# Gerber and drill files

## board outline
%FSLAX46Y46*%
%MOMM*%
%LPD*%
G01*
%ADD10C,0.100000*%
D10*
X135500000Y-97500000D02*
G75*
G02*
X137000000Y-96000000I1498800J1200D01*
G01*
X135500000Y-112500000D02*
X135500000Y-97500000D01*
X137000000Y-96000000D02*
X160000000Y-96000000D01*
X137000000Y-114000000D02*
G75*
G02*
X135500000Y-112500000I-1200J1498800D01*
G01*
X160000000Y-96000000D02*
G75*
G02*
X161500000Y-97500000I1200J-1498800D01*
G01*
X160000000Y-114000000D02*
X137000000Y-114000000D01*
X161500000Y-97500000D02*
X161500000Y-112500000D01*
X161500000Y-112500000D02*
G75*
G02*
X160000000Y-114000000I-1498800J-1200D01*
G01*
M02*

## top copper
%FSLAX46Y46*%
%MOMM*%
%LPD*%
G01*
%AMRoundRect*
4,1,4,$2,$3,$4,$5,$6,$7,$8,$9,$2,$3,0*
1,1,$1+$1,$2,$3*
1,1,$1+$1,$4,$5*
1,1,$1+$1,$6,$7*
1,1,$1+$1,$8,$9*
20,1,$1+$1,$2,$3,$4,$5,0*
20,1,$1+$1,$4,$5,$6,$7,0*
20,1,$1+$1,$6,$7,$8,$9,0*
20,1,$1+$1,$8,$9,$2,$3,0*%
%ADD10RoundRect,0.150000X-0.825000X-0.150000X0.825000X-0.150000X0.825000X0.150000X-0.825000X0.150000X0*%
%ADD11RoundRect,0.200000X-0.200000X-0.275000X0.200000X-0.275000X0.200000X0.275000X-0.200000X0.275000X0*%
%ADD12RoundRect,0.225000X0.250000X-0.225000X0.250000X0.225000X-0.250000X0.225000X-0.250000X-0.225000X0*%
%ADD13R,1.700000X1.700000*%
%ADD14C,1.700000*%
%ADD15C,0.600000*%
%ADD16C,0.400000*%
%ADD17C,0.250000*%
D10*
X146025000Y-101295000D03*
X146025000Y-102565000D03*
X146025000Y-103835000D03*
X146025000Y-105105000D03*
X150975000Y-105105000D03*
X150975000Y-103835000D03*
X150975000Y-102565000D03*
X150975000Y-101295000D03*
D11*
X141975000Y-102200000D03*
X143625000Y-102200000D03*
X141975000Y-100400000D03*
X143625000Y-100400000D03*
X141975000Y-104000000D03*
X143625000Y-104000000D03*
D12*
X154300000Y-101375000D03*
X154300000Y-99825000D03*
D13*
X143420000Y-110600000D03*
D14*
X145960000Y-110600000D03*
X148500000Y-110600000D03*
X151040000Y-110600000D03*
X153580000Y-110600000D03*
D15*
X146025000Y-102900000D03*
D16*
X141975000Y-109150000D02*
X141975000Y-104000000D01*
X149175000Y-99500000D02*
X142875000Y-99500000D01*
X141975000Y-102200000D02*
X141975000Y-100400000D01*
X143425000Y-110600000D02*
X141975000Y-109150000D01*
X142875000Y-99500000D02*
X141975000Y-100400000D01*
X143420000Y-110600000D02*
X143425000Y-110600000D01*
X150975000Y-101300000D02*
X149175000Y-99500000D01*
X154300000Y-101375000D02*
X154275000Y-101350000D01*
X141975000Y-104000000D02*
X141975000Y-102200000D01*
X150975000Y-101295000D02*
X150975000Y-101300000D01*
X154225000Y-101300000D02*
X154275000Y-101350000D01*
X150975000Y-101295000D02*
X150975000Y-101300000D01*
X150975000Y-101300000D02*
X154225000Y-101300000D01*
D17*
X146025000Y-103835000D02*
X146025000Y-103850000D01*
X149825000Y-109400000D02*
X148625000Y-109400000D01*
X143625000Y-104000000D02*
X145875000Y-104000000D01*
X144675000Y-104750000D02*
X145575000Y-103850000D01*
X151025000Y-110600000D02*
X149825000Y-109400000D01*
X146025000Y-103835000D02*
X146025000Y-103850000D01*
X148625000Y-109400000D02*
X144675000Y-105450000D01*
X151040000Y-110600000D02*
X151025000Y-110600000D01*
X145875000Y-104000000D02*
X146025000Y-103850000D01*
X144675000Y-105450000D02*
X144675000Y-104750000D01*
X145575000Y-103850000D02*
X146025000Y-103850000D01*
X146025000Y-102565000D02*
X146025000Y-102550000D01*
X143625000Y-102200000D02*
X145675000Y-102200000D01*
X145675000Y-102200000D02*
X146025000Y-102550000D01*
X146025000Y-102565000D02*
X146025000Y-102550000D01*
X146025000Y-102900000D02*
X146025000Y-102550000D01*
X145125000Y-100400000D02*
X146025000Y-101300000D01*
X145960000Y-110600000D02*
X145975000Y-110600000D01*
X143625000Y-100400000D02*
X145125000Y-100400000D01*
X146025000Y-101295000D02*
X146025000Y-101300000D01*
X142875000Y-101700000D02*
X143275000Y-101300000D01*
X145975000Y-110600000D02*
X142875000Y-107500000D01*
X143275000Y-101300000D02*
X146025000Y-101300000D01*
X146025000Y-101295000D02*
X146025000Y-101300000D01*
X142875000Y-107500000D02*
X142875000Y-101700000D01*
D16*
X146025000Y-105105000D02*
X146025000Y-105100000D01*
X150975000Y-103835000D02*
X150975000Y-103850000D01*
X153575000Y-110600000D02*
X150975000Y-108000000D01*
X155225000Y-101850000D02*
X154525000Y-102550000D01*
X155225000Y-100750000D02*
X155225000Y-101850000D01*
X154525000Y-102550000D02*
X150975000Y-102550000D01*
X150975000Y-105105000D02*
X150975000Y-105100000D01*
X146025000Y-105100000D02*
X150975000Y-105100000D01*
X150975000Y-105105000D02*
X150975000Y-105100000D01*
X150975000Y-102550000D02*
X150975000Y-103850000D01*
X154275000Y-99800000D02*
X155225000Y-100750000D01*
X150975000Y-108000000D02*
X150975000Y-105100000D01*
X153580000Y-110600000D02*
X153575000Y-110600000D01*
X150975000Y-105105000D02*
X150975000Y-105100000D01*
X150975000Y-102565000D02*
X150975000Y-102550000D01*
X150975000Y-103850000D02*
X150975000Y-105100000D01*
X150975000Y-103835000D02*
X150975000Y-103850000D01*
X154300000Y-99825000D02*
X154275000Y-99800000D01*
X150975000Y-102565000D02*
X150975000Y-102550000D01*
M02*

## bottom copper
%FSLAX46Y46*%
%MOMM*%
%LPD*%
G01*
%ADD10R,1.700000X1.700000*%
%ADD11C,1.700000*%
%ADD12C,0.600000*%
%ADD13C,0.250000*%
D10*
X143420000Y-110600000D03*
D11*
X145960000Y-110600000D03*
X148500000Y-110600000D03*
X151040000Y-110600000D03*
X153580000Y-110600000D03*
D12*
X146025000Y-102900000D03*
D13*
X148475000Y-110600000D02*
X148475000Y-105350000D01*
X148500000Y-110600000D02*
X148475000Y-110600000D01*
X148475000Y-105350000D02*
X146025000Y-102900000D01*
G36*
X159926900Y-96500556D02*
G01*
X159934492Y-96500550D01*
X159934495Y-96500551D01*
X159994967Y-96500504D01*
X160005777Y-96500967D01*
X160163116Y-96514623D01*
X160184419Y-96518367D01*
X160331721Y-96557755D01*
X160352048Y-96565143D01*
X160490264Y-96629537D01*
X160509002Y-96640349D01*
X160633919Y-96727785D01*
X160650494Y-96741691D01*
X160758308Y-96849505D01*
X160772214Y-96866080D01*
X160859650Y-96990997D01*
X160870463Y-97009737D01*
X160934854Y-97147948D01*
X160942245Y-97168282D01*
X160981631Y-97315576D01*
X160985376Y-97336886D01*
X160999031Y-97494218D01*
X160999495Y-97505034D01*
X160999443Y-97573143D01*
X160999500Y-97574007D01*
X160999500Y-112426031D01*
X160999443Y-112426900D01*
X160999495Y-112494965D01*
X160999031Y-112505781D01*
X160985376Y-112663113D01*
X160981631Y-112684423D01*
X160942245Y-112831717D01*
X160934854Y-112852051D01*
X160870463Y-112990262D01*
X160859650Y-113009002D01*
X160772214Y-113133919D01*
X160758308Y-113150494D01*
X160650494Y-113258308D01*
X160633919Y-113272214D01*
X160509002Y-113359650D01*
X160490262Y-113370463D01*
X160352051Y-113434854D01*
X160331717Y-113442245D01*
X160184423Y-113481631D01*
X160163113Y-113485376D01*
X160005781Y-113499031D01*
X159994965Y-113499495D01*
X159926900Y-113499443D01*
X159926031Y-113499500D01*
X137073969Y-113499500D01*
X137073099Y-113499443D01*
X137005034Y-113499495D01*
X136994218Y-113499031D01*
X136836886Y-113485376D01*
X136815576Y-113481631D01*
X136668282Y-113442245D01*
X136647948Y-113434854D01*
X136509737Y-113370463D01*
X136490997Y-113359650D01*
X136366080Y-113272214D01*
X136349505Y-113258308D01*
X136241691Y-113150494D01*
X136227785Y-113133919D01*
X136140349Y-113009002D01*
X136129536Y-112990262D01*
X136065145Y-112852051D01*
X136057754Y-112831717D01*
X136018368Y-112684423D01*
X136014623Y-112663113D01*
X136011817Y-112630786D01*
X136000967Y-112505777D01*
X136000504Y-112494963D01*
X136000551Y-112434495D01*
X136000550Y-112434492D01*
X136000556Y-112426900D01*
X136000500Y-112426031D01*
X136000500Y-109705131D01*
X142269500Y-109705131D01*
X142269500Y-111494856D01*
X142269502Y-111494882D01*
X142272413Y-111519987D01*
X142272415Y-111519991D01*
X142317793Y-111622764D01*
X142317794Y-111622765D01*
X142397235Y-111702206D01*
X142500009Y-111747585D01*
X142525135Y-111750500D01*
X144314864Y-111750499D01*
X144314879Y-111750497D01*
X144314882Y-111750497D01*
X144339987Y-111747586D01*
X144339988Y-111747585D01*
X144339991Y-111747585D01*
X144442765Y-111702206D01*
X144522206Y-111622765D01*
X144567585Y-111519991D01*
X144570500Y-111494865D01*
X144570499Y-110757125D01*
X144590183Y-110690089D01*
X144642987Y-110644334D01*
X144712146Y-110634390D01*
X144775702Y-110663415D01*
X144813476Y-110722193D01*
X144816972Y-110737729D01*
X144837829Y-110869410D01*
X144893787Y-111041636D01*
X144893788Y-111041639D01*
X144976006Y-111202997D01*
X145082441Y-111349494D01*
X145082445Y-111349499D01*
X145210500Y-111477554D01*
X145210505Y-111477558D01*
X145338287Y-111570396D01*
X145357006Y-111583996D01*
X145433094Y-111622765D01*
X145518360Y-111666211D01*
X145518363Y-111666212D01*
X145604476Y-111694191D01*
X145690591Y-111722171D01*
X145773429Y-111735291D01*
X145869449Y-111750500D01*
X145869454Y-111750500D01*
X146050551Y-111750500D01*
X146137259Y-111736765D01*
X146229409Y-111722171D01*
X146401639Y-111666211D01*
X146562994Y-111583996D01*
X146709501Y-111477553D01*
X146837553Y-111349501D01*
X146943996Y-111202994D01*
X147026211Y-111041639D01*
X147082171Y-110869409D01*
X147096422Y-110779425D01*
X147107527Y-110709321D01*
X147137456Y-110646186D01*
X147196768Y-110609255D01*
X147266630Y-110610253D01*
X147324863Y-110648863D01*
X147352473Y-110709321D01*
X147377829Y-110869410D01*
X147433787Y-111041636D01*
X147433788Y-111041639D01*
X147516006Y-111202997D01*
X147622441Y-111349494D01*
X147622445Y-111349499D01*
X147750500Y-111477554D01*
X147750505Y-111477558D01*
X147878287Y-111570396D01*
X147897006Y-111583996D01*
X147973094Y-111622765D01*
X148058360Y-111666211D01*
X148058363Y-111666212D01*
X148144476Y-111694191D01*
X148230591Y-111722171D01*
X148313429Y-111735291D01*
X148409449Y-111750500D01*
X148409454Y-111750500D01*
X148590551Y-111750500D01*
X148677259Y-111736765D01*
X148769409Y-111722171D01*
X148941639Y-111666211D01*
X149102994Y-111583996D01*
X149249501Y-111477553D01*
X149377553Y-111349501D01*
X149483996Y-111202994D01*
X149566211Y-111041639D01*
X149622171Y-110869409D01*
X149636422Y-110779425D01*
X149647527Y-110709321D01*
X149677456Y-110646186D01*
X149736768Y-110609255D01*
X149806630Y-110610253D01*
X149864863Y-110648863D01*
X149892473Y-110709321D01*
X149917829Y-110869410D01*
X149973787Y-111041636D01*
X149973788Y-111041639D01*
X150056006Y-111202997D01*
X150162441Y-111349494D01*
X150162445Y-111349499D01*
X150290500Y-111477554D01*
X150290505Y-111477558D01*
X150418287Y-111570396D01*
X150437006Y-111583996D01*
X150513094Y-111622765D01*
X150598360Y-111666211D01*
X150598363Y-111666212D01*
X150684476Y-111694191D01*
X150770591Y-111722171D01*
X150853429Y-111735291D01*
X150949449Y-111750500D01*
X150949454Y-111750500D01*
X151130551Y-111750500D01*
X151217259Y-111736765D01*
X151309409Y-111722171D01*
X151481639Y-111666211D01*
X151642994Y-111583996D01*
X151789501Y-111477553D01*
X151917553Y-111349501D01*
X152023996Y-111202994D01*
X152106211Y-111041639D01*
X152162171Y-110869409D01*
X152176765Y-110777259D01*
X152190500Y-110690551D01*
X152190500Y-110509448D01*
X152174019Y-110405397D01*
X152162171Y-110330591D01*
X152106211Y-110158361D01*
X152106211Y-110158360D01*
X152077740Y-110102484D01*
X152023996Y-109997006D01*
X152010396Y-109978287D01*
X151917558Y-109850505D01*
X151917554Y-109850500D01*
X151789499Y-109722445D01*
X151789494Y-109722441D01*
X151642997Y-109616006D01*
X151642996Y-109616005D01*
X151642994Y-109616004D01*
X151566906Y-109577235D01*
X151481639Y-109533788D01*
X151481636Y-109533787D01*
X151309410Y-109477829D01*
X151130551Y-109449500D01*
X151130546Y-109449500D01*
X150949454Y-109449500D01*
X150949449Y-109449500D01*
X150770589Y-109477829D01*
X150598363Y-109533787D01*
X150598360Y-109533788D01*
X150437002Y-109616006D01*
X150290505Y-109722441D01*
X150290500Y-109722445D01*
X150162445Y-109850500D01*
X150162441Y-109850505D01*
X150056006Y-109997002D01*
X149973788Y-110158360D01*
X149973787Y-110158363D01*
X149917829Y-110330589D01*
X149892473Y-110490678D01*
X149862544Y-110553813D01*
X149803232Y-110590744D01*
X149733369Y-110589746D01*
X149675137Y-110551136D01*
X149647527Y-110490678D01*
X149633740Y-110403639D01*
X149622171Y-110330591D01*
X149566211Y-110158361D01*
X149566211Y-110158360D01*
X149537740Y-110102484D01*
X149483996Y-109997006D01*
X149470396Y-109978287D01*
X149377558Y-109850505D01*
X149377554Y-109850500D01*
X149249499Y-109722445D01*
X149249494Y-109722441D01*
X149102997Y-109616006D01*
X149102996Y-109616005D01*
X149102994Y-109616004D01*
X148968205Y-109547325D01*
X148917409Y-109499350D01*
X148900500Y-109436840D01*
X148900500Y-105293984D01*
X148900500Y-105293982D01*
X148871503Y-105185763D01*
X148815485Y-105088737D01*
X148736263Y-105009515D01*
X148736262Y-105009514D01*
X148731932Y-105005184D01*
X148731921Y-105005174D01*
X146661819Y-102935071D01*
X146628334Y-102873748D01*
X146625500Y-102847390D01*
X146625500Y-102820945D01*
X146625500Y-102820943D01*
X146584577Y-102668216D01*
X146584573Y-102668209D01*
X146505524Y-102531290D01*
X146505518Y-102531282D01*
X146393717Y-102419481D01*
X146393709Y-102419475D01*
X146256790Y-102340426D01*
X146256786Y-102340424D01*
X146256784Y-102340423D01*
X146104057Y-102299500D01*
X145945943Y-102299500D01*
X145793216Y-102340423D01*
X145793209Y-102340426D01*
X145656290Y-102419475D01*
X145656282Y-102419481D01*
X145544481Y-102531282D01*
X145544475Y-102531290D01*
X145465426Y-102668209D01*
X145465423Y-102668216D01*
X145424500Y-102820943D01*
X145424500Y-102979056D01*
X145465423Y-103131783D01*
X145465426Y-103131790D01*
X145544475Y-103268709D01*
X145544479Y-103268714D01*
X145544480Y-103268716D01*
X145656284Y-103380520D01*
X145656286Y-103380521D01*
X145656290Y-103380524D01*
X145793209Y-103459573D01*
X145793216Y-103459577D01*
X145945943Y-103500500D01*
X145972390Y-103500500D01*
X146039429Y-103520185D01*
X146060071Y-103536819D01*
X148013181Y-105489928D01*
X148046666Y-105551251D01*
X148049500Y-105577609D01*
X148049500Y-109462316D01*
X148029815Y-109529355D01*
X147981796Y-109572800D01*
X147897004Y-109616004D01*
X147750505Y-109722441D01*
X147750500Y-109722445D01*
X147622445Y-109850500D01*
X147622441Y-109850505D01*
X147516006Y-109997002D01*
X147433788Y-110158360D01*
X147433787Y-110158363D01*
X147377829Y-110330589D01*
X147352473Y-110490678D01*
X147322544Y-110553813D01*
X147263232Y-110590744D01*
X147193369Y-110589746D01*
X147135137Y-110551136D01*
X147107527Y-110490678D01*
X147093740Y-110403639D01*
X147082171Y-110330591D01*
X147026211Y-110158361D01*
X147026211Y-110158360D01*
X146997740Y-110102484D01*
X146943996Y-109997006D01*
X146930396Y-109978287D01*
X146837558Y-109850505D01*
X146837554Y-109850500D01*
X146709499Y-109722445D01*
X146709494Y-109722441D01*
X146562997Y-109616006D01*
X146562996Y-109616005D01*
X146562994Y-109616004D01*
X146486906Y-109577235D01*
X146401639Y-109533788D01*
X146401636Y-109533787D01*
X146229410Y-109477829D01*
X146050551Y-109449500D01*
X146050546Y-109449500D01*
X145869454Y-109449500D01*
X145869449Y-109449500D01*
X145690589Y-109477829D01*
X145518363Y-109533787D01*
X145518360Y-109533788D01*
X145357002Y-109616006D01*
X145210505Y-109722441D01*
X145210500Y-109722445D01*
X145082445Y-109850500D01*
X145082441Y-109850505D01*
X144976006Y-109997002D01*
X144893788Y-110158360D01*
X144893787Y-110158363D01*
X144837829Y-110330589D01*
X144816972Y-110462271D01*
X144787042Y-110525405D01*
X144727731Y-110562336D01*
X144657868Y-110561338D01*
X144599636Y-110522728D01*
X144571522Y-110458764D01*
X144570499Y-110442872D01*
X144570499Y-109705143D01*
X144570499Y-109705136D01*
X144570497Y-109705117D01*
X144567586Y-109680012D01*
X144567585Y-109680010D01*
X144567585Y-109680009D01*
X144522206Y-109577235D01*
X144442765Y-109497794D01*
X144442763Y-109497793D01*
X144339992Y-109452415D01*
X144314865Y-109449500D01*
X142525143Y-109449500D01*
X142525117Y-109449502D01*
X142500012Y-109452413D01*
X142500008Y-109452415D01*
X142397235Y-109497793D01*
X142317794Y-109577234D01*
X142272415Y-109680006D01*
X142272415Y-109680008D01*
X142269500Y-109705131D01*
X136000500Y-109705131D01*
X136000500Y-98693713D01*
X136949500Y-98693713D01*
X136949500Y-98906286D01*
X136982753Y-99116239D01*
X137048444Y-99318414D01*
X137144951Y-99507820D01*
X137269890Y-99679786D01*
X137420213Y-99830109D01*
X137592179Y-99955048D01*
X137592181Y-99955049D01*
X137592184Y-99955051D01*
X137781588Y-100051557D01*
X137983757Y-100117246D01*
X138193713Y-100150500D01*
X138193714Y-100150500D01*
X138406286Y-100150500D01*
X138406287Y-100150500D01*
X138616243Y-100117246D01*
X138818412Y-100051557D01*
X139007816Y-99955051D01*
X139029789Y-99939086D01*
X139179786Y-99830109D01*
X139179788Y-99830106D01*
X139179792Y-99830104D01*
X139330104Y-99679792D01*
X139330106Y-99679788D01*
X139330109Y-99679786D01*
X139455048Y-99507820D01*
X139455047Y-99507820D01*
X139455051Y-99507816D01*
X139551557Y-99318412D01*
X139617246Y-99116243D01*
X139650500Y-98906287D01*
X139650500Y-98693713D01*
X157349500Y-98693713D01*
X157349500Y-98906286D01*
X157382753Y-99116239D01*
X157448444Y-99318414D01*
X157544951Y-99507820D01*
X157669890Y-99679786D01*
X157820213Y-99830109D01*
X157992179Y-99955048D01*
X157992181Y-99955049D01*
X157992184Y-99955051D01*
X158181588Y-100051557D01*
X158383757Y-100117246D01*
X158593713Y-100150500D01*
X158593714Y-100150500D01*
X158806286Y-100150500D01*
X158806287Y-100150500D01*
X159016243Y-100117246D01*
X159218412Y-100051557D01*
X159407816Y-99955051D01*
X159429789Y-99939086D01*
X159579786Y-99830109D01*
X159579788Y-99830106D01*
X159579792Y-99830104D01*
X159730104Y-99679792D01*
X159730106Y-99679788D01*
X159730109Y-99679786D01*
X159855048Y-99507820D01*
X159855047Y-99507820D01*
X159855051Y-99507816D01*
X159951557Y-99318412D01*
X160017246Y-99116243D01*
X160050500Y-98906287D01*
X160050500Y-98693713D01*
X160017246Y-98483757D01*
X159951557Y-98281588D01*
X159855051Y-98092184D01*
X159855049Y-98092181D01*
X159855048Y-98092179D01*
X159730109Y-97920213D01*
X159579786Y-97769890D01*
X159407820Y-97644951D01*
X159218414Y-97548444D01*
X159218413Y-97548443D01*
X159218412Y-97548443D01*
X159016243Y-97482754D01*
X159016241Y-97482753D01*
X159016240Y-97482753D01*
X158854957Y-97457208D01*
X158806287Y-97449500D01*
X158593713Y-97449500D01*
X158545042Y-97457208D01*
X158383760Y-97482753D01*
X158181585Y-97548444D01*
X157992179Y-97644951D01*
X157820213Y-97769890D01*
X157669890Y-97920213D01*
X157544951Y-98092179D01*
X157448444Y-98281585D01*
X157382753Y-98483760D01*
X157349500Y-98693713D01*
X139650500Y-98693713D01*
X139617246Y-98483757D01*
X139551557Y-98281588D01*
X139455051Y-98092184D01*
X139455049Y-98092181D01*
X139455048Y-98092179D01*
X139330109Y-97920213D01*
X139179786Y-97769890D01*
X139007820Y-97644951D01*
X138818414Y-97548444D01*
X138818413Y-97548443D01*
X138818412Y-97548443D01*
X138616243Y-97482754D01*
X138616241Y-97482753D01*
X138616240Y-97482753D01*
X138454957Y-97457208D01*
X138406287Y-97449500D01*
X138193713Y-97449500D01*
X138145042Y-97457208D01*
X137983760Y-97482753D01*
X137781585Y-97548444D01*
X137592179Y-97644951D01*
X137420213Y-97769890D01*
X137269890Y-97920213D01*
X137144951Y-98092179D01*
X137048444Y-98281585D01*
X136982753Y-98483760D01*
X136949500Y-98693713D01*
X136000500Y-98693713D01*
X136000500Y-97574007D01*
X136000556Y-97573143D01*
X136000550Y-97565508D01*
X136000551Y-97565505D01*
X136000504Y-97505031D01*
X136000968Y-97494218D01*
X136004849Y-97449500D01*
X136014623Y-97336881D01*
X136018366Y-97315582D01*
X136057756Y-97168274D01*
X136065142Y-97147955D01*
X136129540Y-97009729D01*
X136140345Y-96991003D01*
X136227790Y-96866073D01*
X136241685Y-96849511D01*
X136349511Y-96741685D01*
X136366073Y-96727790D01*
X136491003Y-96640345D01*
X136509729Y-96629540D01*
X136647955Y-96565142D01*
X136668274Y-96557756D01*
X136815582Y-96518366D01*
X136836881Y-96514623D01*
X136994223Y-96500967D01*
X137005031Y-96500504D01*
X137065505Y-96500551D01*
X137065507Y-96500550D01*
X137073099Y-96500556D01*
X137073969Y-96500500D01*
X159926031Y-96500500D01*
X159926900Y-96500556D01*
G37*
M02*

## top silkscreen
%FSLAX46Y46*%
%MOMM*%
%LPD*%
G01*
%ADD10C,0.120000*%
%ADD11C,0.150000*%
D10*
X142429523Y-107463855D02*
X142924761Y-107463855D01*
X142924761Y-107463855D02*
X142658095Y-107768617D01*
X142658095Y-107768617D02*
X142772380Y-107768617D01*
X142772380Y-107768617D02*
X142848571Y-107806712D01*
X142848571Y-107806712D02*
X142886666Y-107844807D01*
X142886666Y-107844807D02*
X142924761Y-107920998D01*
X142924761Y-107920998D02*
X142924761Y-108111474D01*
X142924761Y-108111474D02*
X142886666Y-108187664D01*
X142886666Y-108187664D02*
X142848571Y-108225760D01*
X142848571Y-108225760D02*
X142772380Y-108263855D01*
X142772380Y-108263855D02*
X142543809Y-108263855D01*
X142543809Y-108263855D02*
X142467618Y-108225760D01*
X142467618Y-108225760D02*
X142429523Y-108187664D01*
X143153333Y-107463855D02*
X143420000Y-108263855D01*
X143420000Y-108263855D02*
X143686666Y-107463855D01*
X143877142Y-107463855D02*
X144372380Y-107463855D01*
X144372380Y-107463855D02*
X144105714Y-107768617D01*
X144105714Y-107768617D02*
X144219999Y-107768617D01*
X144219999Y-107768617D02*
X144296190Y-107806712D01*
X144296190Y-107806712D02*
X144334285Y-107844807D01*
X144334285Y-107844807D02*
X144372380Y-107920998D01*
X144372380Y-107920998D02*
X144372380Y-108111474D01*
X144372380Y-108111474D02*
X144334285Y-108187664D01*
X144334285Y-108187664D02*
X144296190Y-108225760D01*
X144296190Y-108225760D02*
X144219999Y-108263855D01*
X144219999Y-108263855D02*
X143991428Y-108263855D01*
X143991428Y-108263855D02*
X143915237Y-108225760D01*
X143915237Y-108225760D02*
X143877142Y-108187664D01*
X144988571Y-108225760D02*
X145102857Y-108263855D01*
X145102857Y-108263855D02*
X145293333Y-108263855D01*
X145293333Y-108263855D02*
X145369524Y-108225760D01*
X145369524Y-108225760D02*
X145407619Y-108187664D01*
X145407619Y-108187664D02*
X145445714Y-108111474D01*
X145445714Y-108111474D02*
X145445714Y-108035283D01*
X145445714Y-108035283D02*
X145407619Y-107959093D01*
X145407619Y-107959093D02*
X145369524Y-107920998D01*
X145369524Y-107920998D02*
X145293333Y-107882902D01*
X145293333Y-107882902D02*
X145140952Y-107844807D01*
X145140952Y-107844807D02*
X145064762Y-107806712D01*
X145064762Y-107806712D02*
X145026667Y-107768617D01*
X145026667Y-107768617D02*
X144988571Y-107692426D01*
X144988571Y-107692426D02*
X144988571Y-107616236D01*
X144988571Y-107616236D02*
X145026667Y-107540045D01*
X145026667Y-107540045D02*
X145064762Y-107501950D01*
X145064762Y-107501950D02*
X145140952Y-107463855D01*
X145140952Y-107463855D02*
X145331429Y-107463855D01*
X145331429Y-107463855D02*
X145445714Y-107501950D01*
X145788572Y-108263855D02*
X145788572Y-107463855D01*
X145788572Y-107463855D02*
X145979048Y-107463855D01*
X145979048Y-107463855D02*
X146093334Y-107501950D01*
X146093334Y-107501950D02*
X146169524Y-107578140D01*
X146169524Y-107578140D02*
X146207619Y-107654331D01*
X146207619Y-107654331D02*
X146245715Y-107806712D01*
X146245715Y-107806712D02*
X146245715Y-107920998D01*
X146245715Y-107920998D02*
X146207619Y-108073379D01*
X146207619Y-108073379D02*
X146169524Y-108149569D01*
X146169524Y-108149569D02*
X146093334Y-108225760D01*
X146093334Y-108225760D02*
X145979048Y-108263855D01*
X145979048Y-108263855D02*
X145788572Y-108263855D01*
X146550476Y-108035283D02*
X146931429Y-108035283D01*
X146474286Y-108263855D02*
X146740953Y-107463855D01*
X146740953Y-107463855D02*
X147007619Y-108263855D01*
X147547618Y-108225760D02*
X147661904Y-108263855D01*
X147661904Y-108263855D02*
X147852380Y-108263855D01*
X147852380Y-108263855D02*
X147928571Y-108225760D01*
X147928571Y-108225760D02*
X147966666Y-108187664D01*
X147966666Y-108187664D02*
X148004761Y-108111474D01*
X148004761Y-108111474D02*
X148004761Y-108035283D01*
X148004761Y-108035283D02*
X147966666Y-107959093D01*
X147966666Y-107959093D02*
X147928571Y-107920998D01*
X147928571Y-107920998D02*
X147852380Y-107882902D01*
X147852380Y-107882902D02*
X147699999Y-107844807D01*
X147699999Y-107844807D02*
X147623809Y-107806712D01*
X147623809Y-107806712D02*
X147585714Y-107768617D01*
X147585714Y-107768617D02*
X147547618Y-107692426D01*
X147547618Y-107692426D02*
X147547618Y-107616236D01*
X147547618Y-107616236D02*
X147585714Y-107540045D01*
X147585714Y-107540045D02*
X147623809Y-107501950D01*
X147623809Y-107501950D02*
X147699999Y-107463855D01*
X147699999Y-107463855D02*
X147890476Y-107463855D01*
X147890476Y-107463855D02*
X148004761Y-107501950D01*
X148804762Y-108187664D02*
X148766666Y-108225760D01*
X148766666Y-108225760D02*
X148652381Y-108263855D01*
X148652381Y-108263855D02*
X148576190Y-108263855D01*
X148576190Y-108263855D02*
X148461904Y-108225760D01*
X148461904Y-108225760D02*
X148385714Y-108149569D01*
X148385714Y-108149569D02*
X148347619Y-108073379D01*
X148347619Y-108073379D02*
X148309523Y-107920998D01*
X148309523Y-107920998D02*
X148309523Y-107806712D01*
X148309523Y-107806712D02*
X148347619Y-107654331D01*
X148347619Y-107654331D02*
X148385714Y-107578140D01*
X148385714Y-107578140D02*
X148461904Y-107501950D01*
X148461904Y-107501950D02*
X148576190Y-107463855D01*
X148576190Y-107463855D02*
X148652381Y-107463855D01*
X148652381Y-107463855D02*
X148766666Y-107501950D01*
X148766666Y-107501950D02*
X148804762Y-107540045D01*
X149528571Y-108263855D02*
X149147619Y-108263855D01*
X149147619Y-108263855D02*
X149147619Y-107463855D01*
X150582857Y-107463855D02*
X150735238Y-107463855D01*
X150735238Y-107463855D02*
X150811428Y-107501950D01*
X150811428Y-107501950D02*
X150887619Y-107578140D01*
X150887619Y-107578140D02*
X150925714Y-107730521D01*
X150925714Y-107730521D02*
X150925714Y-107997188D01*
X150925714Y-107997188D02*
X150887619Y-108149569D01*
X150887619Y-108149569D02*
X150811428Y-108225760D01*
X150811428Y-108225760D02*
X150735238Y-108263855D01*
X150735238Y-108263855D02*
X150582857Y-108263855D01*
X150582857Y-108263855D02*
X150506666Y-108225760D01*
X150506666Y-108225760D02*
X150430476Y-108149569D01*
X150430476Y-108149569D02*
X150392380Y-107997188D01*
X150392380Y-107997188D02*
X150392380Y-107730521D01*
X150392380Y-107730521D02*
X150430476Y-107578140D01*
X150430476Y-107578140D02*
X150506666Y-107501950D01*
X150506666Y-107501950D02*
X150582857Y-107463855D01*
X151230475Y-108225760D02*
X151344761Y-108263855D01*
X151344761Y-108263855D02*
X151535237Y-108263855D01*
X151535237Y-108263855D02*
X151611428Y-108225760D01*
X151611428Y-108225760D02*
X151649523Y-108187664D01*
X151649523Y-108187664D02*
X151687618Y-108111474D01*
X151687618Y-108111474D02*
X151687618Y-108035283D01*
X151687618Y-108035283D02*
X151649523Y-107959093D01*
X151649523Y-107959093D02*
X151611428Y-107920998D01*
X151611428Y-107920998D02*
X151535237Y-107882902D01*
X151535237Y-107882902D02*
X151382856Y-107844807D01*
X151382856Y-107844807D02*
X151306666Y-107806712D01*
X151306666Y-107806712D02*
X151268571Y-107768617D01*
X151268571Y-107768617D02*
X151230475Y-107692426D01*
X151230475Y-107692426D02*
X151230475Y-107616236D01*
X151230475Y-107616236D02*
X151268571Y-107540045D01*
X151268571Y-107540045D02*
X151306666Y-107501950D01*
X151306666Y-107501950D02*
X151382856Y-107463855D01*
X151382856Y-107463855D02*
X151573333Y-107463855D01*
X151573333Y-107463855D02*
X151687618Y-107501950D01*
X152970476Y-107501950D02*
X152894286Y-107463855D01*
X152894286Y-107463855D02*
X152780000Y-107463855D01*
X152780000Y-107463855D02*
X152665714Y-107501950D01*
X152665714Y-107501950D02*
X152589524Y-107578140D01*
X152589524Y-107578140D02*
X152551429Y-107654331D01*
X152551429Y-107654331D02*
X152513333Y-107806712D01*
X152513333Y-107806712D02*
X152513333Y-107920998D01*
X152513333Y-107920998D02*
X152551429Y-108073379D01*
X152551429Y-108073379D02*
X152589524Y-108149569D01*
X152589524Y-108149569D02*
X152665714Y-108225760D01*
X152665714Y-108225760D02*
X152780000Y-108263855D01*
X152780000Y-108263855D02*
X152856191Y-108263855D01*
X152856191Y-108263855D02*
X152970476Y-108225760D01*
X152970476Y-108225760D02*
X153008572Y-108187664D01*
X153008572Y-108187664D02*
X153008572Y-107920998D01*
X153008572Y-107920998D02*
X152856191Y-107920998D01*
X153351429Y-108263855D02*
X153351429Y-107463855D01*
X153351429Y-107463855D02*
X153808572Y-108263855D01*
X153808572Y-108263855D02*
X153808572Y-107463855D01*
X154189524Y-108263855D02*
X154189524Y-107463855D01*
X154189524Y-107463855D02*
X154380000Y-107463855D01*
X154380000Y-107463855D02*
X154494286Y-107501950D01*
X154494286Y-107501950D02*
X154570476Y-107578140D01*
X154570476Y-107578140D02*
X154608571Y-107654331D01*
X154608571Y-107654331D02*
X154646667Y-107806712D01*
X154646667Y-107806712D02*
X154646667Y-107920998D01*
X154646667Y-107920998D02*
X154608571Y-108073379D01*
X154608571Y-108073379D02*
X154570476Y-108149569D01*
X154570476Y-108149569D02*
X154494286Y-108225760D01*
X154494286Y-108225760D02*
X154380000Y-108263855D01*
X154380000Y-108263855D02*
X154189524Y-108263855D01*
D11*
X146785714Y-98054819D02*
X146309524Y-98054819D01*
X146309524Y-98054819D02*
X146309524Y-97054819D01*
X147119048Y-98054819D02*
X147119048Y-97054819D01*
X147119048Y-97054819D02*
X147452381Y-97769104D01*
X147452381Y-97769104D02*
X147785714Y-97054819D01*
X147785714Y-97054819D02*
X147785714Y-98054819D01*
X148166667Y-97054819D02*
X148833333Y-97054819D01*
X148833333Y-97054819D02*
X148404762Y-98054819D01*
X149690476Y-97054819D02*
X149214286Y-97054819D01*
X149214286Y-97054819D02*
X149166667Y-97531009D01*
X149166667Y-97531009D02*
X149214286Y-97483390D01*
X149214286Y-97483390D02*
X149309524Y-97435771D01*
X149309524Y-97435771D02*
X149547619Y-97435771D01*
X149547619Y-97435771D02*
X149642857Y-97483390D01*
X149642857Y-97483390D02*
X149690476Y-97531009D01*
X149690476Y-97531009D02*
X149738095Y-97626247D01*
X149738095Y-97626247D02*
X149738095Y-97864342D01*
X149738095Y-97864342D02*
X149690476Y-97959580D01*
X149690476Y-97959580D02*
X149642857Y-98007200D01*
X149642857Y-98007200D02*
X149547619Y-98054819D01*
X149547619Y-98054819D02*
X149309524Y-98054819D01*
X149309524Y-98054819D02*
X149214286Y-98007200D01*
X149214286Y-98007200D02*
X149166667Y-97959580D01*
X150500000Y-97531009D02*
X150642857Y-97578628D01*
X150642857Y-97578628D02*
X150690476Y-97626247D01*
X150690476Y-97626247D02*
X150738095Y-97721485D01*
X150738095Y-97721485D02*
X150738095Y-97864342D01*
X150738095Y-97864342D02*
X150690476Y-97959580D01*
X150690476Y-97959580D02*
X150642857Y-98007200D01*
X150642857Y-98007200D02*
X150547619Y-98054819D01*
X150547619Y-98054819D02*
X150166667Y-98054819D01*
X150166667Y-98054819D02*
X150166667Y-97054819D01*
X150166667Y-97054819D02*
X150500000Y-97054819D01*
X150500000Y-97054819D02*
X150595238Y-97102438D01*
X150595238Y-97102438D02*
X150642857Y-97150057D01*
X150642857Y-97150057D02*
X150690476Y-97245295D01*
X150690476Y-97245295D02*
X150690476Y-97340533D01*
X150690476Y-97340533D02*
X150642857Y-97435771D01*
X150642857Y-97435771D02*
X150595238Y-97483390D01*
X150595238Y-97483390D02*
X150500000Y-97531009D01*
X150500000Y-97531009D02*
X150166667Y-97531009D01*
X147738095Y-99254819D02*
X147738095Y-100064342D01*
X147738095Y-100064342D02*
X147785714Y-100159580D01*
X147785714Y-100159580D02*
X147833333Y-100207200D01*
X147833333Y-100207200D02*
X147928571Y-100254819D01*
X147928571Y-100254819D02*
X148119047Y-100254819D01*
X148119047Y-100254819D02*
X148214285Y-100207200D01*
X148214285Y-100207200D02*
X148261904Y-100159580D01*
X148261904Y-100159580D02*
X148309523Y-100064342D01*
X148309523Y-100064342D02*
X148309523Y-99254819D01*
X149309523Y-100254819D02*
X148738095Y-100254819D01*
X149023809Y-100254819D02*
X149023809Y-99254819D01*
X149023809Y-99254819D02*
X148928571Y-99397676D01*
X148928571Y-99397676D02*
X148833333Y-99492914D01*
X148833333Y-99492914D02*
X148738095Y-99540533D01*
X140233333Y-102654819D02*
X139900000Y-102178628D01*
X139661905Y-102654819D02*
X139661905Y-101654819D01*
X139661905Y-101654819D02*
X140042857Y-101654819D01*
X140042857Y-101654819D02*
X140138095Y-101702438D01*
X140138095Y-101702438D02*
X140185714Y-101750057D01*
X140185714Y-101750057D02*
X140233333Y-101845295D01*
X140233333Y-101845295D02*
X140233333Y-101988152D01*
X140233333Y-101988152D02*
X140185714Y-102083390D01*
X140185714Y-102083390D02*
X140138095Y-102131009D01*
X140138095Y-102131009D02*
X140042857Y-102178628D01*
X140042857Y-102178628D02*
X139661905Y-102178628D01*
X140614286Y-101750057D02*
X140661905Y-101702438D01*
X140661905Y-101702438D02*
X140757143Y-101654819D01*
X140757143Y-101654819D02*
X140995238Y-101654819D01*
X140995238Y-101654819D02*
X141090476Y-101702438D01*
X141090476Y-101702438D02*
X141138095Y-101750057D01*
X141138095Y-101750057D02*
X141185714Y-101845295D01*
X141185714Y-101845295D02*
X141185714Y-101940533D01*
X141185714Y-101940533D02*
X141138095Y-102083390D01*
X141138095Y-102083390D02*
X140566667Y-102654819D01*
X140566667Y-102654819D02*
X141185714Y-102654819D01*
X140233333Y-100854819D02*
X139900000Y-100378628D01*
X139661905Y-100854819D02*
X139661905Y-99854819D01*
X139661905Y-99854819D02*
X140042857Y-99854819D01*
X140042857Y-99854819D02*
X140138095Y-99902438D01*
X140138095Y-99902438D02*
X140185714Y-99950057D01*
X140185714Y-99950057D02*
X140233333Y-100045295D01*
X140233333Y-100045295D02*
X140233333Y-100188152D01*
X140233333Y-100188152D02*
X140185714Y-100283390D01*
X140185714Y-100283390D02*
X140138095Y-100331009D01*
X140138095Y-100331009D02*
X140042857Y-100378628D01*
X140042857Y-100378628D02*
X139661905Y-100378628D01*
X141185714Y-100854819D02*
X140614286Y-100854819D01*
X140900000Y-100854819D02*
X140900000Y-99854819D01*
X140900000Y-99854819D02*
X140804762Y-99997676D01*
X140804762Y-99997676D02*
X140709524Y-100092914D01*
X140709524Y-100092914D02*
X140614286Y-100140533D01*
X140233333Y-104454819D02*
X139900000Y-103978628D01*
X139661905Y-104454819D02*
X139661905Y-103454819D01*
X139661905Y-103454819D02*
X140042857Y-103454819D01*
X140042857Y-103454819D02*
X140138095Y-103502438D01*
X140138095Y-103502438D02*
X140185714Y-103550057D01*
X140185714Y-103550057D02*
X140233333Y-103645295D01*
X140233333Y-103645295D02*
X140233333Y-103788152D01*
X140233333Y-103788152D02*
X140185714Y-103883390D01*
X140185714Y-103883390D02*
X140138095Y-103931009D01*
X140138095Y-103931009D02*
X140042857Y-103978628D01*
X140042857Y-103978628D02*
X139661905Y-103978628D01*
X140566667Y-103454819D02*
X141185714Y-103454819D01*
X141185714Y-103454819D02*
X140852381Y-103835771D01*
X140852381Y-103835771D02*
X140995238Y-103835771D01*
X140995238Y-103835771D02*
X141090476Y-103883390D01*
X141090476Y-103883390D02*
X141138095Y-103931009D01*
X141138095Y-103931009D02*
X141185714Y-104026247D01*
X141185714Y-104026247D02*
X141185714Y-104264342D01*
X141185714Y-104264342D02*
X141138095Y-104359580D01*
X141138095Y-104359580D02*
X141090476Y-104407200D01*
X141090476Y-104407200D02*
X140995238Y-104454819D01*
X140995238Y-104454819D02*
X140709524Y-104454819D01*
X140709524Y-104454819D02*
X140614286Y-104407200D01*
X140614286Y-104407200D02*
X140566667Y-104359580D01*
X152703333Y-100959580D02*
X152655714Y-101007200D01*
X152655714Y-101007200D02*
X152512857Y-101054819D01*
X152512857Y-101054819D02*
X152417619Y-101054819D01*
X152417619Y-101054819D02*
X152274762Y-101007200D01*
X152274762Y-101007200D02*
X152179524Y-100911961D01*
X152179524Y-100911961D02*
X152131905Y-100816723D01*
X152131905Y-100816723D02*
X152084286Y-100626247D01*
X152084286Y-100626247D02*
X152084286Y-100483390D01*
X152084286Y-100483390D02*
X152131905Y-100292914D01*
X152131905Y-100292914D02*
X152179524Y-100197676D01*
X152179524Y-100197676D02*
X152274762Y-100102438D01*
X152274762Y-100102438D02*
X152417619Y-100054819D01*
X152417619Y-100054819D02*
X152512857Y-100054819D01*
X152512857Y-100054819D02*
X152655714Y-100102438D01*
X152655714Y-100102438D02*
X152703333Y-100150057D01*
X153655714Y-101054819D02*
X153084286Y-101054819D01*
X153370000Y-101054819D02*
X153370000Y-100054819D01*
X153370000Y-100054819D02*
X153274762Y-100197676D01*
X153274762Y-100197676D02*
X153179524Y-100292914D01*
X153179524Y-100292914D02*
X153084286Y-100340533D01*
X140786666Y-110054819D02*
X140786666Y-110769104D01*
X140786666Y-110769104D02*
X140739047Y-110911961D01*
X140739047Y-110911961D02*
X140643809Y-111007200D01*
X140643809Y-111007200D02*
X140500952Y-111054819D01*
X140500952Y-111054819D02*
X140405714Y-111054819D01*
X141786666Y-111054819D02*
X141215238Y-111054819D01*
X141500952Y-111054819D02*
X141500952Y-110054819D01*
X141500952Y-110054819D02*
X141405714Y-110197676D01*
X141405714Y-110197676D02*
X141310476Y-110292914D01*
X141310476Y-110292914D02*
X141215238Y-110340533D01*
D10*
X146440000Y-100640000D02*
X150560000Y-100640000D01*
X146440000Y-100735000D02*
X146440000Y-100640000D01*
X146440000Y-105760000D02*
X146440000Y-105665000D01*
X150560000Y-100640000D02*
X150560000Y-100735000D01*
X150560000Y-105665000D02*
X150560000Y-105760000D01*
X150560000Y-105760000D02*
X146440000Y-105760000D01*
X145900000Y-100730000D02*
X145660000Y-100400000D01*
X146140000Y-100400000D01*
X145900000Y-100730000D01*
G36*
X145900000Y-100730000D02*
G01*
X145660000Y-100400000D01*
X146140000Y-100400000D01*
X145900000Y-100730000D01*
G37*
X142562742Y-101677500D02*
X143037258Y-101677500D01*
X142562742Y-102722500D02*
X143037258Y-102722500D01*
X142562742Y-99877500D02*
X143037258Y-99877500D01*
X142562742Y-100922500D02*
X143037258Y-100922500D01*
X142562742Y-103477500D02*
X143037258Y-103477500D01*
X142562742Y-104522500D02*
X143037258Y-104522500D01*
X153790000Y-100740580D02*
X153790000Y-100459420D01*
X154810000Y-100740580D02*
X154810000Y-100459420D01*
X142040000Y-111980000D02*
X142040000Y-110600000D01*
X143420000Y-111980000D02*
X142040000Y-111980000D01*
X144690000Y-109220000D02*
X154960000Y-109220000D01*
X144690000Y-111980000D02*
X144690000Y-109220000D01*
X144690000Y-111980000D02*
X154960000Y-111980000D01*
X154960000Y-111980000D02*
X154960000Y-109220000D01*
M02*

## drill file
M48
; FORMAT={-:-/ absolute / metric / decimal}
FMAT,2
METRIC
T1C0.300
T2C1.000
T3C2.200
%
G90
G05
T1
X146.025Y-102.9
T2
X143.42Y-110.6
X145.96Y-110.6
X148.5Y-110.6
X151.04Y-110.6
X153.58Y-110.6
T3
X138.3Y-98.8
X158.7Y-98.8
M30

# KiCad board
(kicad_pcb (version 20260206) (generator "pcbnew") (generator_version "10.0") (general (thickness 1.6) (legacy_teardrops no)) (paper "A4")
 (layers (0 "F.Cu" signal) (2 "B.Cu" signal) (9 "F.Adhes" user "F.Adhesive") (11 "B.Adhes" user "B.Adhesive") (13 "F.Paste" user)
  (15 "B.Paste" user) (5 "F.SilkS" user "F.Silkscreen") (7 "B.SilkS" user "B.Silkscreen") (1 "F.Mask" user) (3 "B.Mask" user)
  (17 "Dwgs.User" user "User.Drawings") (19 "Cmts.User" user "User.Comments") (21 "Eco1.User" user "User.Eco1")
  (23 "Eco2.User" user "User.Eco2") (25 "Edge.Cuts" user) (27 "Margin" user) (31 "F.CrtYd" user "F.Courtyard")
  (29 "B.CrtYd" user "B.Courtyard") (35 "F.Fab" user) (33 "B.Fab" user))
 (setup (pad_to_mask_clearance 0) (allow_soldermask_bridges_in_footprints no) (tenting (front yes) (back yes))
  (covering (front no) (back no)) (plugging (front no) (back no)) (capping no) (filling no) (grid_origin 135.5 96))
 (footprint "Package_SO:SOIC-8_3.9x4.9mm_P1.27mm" (layer "F.Cu") (at 148.5 103.2)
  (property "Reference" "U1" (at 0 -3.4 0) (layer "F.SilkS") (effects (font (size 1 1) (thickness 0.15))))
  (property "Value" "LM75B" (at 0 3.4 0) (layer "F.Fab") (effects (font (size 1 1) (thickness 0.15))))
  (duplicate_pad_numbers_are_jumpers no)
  (fp_line (start -2.06 -2.56) (end 2.06 -2.56) (stroke (width 0.12) (type solid)) (layer "F.SilkS"))
  (fp_line (start -2.06 -2.465) (end -2.06 -2.56) (stroke (width 0.12) (type solid)) (layer "F.SilkS"))
  (fp_line (start -2.06 2.56) (end -2.06 2.465) (stroke (width 0.12) (type solid)) (layer "F.SilkS"))
  (fp_line (start 2.06 -2.56) (end 2.06 -2.465) (stroke (width 0.12) (type solid)) (layer "F.SilkS"))
  (fp_line (start 2.06 2.465) (end 2.06 2.56) (stroke (width 0.12) (type solid)) (layer "F.SilkS"))
  (fp_line (start 2.06 2.56) (end -2.06 2.56) (stroke (width 0.12) (type solid)) (layer "F.SilkS"))
  (fp_poly (pts (xy -2.6 -2.47) (xy -2.84 -2.8) (xy -2.36 -2.8)) (stroke (width 0.12) (type solid)) (fill yes) (layer "F.SilkS"))
  (pad "1" smd roundrect (at -2.475 -1.905) (size 1.95 0.6) (layers "F.Cu" "F.Mask" "F.Paste") (roundrect_rratio 0.25) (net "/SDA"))
  (pad "2" smd roundrect (at -2.475 -0.635) (size 1.95 0.6) (layers "F.Cu" "F.Mask" "F.Paste") (roundrect_rratio 0.25) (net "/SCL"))
  (pad "3" smd roundrect (at -2.475 0.635) (size 1.95 0.6) (layers "F.Cu" "F.Mask" "F.Paste") (roundrect_rratio 0.25) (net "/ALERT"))
  (pad "4" smd roundrect (at -2.475 1.905) (size 1.95 0.6) (layers "F.Cu" "F.Mask" "F.Paste") (roundrect_rratio 0.25) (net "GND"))
  (pad "5" smd roundrect (at 2.475 1.905) (size 1.95 0.6) (layers "F.Cu" "F.Mask" "F.Paste") (roundrect_rratio 0.25) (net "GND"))
  (pad "6" smd roundrect (at 2.475 0.635) (size 1.95 0.6) (layers "F.Cu" "F.Mask" "F.Paste") (roundrect_rratio 0.25) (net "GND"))
  (pad "7" smd roundrect (at 2.475 -0.635) (size 1.95 0.6) (layers "F.Cu" "F.Mask" "F.Paste") (roundrect_rratio 0.25) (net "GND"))
  (pad "8" smd roundrect (at 2.475 -1.905) (size 1.95 0.6) (layers "F.Cu" "F.Mask" "F.Paste") (roundrect_rratio 0.25) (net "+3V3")))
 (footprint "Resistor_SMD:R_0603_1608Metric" (layer "F.Cu") (at 142.8 102.2)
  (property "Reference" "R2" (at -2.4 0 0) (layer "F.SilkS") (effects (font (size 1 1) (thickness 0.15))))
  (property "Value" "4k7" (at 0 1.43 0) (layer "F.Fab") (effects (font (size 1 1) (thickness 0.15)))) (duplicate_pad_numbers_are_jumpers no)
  (fp_line (start -0.237258 -0.5225) (end 0.237258 -0.5225) (stroke (width 0.12) (type solid)) (layer "F.SilkS"))
  (fp_line (start -0.237258 0.5225) (end 0.237258 0.5225) (stroke (width 0.12) (type solid)) (layer "F.SilkS"))
  (pad "1" smd roundrect (at -0.825 0) (size 0.8 0.95) (layers "F.Cu" "F.Mask" "F.Paste") (roundrect_rratio 0.25) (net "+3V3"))
  (pad "2" smd roundrect (at 0.825 0) (size 0.8 0.95) (layers "F.Cu" "F.Mask" "F.Paste") (roundrect_rratio 0.25) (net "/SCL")))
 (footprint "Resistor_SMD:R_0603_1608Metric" (layer "F.Cu") (at 142.8 100.4)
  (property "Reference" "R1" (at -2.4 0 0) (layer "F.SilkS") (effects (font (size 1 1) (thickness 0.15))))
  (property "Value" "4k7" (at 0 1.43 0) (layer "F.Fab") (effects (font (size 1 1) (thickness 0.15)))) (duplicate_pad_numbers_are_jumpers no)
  (fp_line (start -0.237258 -0.5225) (end 0.237258 -0.5225) (stroke (width 0.12) (type solid)) (layer "F.SilkS"))
  (fp_line (start -0.237258 0.5225) (end 0.237258 0.5225) (stroke (width 0.12) (type solid)) (layer "F.SilkS"))
  (pad "1" smd roundrect (at -0.825 0) (size 0.8 0.95) (layers "F.Cu" "F.Mask" "F.Paste") (roundrect_rratio 0.25) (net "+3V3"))
  (pad "2" smd roundrect (at 0.825 0) (size 0.8 0.95) (layers "F.Cu" "F.Mask" "F.Paste") (roundrect_rratio 0.25) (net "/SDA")))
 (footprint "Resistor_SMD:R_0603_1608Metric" (layer "F.Cu") (at 142.8 104)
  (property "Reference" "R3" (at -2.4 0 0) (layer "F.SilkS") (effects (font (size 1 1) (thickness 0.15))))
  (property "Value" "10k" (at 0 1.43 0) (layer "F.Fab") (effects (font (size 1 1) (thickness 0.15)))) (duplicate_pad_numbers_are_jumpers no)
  (fp_line (start -0.237258 -0.5225) (end 0.237258 -0.5225) (stroke (width 0.12) (type solid)) (layer "F.SilkS"))
  (fp_line (start -0.237258 0.5225) (end 0.237258 0.5225) (stroke (width 0.12) (type solid)) (layer "F.SilkS"))
  (pad "1" smd roundrect (at -0.825 0) (size 0.8 0.95) (layers "F.Cu" "F.Mask" "F.Paste") (roundrect_rratio 0.25) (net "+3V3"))
  (pad "2" smd roundrect (at 0.825 0) (size 0.8 0.95) (layers "F.Cu" "F.Mask" "F.Paste") (roundrect_rratio 0.25) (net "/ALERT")))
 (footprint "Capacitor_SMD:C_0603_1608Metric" (layer "F.Cu") (at 154.3 100.6 90)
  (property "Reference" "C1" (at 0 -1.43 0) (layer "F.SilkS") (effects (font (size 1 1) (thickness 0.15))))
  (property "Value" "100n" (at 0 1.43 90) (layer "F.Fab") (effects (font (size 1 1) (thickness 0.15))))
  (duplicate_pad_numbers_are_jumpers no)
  (fp_line (start -0.14058 -0.51) (end 0.14058 -0.51) (stroke (width 0.12) (type solid)) (layer "F.SilkS"))
  (fp_line (start -0.14058 0.51) (end 0.14058 0.51) (stroke (width 0.12) (type solid)) (layer "F.SilkS"))
  (pad "1" smd roundrect (at -0.775 0 90) (size 0.9 0.95) (layers "F.Cu" "F.Mask" "F.Paste") (roundrect_rratio 0.25) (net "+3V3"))
  (pad "2" smd roundrect (at 0.775 0 90) (size 0.9 0.95) (layers "F.Cu" "F.Mask" "F.Paste") (roundrect_rratio 0.25) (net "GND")))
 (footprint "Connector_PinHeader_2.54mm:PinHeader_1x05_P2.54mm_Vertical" (layer "F.Cu") (at 143.42 110.6 90)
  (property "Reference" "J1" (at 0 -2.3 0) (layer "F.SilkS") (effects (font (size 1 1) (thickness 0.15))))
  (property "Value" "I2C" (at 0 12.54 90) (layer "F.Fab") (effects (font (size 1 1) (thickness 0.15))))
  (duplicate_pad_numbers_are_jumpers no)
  (fp_line (start -1.38 -1.38) (end 0 -1.38) (stroke (width 0.12) (type solid)) (layer "F.SilkS"))
  (fp_line (start -1.38 0) (end -1.38 -1.38) (stroke (width 0.12) (type solid)) (layer "F.SilkS"))
  (fp_line (start 1.38 1.27) (end 1.38 11.54) (stroke (width 0.12) (type solid)) (layer "F.SilkS"))
  (fp_line (start -1.38 1.27) (end 1.38 1.27) (stroke (width 0.12) (type solid)) (layer "F.SilkS"))
  (fp_line (start -1.38 1.27) (end -1.38 11.54) (stroke (width 0.12) (type solid)) (layer "F.SilkS"))
  (fp_line (start -1.38 11.54) (end 1.38 11.54) (stroke (width 0.12) (type solid)) (layer "F.SilkS"))
  (pad "1" thru_hole rect (at 0 0 90) (size 1.7 1.7) (drill 1) (layers "*.Cu" "*.Mask") (remove_unused_layers no) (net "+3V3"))
  (pad "2" thru_hole circle (at 0 2.54 90) (size 1.7 1.7) (drill 1) (layers "*.Cu" "*.Mask") (remove_unused_layers no) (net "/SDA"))
  (pad "3" thru_hole circle (at 0 5.08 90) (size 1.7 1.7) (drill 1) (layers "*.Cu" "*.Mask") (remove_unused_layers no) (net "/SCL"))
  (pad "4" thru_hole circle (at 0 7.62 90) (size 1.7 1.7) (drill 1) (layers "*.Cu" "*.Mask") (remove_unused_layers no) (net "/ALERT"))
  (pad "5" thru_hole circle (at 0 10.16 90) (size 1.7 1.7) (drill 1) (layers "*.Cu" "*.Mask") (remove_unused_layers no) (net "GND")))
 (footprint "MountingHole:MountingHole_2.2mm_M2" (layer "F.Cu") (at 138.3 98.8)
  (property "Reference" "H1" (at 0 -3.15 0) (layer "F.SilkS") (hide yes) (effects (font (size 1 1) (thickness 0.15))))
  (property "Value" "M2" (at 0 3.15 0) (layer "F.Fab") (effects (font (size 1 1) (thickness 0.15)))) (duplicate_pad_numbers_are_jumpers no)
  (pad "" np_thru_hole circle (at 0 0) (size 2.2 2.2) (drill 2.2) (layers "*.Cu" "*.Mask")))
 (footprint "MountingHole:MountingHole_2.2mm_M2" (layer "F.Cu") (at 158.7 98.8)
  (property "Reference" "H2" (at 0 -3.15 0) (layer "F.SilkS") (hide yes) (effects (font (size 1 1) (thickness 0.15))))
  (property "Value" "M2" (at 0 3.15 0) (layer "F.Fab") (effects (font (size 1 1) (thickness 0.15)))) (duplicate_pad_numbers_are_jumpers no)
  (pad "" np_thru_hole circle (at 0 0) (size 2.2 2.2) (drill 2.2) (layers "*.Cu" "*.Mask")))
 (gr_arc (start 135.5 97.5) (mid 135.939 96.439) (end 137 96) (stroke (width 0.1) (type default)) (layer "Edge.Cuts"))
 (gr_line (start 135.5 112.5) (end 135.5 97.5) (stroke (width 0.1) (type default)) (layer "Edge.Cuts"))
 (gr_line (start 137 96) (end 160 96) (stroke (width 0.1) (type default)) (layer "Edge.Cuts"))
 (gr_arc (start 137 114) (mid 135.939 113.561) (end 135.5 112.5) (stroke (width 0.1) (type default)) (layer "Edge.Cuts"))
 (gr_arc (start 160 96) (mid 161.061 96.439) (end 161.5 97.5) (stroke (width 0.1) (type default)) (layer "Edge.Cuts"))
 (gr_line (start 160 114) (end 137 114) (stroke (width 0.1) (type default)) (layer "Edge.Cuts"))
 (gr_line (start 161.5 97.5) (end 161.5 112.5) (stroke (width 0.1) (type default)) (layer "Edge.Cuts"))
 (gr_arc (start 161.5 112.5) (mid 161.061 113.561) (end 160 114) (stroke (width 0.1) (type default)) (layer "Edge.Cuts"))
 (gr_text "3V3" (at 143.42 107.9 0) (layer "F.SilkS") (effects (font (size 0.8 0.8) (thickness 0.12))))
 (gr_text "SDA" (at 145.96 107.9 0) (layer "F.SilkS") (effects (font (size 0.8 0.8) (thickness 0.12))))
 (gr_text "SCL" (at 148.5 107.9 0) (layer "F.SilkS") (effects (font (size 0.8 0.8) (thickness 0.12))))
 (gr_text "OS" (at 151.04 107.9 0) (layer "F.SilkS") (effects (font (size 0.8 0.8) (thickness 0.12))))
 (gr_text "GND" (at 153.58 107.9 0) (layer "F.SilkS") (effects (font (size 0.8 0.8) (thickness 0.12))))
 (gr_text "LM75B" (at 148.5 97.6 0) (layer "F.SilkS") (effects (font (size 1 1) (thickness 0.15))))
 (segment (start 141.975 109.15) (end 141.975 104) (width 0.4) (layer "F.Cu") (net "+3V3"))
 (segment (start 149.175 99.5) (end 142.875 99.5) (width 0.4) (layer "F.Cu") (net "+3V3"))
 (segment (start 141.975 102.2) (end 141.975 100.4) (width 0.4) (layer "F.Cu") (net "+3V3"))
 (segment (start 143.425 110.6) (end 141.975 109.15) (width 0.4) (layer "F.Cu") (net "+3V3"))
 (segment (start 142.875 99.5) (end 141.975 100.4) (width 0.4) (layer "F.Cu") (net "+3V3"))
 (segment (start 143.42 110.6) (end 143.425 110.6) (width 0.4) (layer "F.Cu") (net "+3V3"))
 (segment (start 150.975 101.3) (end 149.175 99.5) (width 0.4) (layer "F.Cu") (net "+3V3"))
 (segment (start 154.3 101.375) (end 154.275 101.35) (width 0.4) (layer "F.Cu") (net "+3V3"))
 (segment (start 141.975 104) (end 141.975 102.2) (width 0.4) (layer "F.Cu") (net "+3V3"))
 (segment (start 150.975 101.295) (end 150.975 101.3) (width 0.4) (layer "F.Cu") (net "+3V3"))
 (segment (start 154.225 101.3) (end 154.275 101.35) (width 0.4) (layer "F.Cu") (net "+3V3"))
 (segment (start 150.975 101.295) (end 150.975 101.3) (width 0.4) (layer "F.Cu") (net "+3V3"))
 (segment (start 150.975 101.3) (end 154.225 101.3) (width 0.4) (layer "F.Cu") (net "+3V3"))
 (segment (start 146.025 103.835) (end 146.025 103.85) (width 0.25) (layer "F.Cu") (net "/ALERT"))
 (segment (start 149.825 109.4) (end 148.625 109.4) (width 0.25) (layer "F.Cu") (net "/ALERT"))
 (segment (start 143.625 104) (end 145.875 104) (width 0.25) (layer "F.Cu") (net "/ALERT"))
 (segment (start 144.675 104.75) (end 145.575 103.85) (width 0.25) (layer "F.Cu") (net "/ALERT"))
 (segment (start 151.025 110.6) (end 149.825 109.4) (width 0.25) (layer "F.Cu") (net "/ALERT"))
 (segment (start 146.025 103.835) (end 146.025 103.85) (width 0.25) (layer "F.Cu") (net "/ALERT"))
 (segment (start 148.625 109.4) (end 144.675 105.45) (width 0.25) (layer "F.Cu") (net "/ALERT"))
 (segment (start 151.04 110.6) (end 151.025 110.6) (width 0.25) (layer "F.Cu") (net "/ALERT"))
 (segment (start 145.875 104) (end 146.025 103.85) (width 0.25) (layer "F.Cu") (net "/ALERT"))
 (segment (start 144.675 105.45) (end 144.675 104.75) (width 0.25) (layer "F.Cu") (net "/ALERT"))
 (segment (start 145.575 103.85) (end 146.025 103.85) (width 0.25) (layer "F.Cu") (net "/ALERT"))
 (segment (start 146.025 102.565) (end 146.025 102.55) (width 0.25) (layer "F.Cu") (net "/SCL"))
 (segment (start 143.625 102.2) (end 145.675 102.2) (width 0.25) (layer "F.Cu") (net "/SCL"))
 (segment (start 145.675 102.2) (end 146.025 102.55) (width 0.25) (layer "F.Cu") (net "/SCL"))
 (segment (start 146.025 102.565) (end 146.025 102.55) (width 0.25) (layer "F.Cu") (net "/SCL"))
 (segment (start 146.025 102.9) (end 146.025 102.55) (width 0.25) (layer "F.Cu") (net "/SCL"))
 (via (at 146.025 102.9) (size 0.6) (drill 0.3) (layers "F.Cu" "B.Cu") (capping no) (covering (front no) (back no))
  (plugging (front no) (back no)) (filling no) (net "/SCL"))
 (segment (start 148.475 110.6) (end 148.475 105.35) (width 0.25) (layer "B.Cu") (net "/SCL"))
 (segment (start 148.5 110.6) (end 148.475 110.6) (width 0.25) (layer "B.Cu") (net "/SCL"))
 (segment (start 148.475 105.35) (end 146.025 102.9) (width 0.25) (layer "B.Cu") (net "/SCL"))
 (segment (start 145.125 100.4) (end 146.025 101.3) (width 0.25) (layer "F.Cu") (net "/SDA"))
 (segment (start 145.96 110.6) (end 145.975 110.6) (width 0.25) (layer "F.Cu") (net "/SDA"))
 (segment (start 143.625 100.4) (end 145.125 100.4) (width 0.25) (layer "F.Cu") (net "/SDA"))
 (segment (start 146.025 101.295) (end 146.025 101.3) (width 0.25) (layer "F.Cu") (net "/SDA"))
 (segment (start 142.875 101.7) (end 143.275 101.3) (width 0.25) (layer "F.Cu") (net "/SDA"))
 (segment (start 145.975 110.6) (end 142.875 107.5) (width 0.25) (layer "F.Cu") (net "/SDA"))
 (segment (start 143.275 101.3) (end 146.025 101.3) (width 0.25) (layer "F.Cu") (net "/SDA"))
 (segment (start 146.025 101.295) (end 146.025 101.3) (width 0.25) (layer "F.Cu") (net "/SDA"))
 (segment (start 142.875 107.5) (end 142.875 101.7) (width 0.25) (layer "F.Cu") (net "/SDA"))
 (segment (start 146.025 105.105) (end 146.025 105.1) (width 0.4) (layer "F.Cu") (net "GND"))
 (segment (start 150.975 103.835) (end 150.975 103.85) (width 0.4) (layer "F.Cu") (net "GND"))
 (segment (start 153.575 110.6) (end 150.975 108) (width 0.4) (layer "F.Cu") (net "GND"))
 (segment (start 155.225 101.85) (end 154.525 102.55) (width 0.4) (layer "F.Cu") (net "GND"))
 (segment (start 155.225 100.75) (end 155.225 101.85) (width 0.4) (layer "F.Cu") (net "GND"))
 (segment (start 154.525 102.55) (end 150.975 102.55) (width 0.4) (layer "F.Cu") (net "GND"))
 (segment (start 150.975 105.105) (end 150.975 105.1) (width 0.4) (layer "F.Cu") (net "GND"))
 (segment (start 146.025 105.1) (end 150.975 105.1) (width 0.4) (layer "F.Cu") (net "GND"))
 (segment (start 150.975 105.105) (end 150.975 105.1) (width 0.4) (layer "F.Cu") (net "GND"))
 (segment (start 150.975 102.55) (end 150.975 103.85) (width 0.4) (layer "F.Cu") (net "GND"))
 (segment (start 154.275 99.8) (end 155.225 100.75) (width 0.4) (layer "F.Cu") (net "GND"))
 (segment (start 150.975 108) (end 150.975 105.1) (width 0.4) (layer "F.Cu") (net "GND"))
 (segment (start 153.58 110.6) (end 153.575 110.6) (width 0.4) (layer "F.Cu") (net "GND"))
 (segment (start 150.975 105.105) (end 150.975 105.1) (width 0.4) (layer "F.Cu") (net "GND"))
 (segment (start 150.975 102.565) (end 150.975 102.55) (width 0.4) (layer "F.Cu") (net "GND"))
 (segment (start 150.975 103.85) (end 150.975 105.1) (width 0.4) (layer "F.Cu") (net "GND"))
 (segment (start 150.975 103.835) (end 150.975 103.85) (width 0.4) (layer "F.Cu") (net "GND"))
 (segment (start 154.3 99.825) (end 154.275 99.8) (width 0.4) (layer "F.Cu") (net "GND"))
 (segment (start 150.975 102.565) (end 150.975 102.55) (width 0.4) (layer "F.Cu") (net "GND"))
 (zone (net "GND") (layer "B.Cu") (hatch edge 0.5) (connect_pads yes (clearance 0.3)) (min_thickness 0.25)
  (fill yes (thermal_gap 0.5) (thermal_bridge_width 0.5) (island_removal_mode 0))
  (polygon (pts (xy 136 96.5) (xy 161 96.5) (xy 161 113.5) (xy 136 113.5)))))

